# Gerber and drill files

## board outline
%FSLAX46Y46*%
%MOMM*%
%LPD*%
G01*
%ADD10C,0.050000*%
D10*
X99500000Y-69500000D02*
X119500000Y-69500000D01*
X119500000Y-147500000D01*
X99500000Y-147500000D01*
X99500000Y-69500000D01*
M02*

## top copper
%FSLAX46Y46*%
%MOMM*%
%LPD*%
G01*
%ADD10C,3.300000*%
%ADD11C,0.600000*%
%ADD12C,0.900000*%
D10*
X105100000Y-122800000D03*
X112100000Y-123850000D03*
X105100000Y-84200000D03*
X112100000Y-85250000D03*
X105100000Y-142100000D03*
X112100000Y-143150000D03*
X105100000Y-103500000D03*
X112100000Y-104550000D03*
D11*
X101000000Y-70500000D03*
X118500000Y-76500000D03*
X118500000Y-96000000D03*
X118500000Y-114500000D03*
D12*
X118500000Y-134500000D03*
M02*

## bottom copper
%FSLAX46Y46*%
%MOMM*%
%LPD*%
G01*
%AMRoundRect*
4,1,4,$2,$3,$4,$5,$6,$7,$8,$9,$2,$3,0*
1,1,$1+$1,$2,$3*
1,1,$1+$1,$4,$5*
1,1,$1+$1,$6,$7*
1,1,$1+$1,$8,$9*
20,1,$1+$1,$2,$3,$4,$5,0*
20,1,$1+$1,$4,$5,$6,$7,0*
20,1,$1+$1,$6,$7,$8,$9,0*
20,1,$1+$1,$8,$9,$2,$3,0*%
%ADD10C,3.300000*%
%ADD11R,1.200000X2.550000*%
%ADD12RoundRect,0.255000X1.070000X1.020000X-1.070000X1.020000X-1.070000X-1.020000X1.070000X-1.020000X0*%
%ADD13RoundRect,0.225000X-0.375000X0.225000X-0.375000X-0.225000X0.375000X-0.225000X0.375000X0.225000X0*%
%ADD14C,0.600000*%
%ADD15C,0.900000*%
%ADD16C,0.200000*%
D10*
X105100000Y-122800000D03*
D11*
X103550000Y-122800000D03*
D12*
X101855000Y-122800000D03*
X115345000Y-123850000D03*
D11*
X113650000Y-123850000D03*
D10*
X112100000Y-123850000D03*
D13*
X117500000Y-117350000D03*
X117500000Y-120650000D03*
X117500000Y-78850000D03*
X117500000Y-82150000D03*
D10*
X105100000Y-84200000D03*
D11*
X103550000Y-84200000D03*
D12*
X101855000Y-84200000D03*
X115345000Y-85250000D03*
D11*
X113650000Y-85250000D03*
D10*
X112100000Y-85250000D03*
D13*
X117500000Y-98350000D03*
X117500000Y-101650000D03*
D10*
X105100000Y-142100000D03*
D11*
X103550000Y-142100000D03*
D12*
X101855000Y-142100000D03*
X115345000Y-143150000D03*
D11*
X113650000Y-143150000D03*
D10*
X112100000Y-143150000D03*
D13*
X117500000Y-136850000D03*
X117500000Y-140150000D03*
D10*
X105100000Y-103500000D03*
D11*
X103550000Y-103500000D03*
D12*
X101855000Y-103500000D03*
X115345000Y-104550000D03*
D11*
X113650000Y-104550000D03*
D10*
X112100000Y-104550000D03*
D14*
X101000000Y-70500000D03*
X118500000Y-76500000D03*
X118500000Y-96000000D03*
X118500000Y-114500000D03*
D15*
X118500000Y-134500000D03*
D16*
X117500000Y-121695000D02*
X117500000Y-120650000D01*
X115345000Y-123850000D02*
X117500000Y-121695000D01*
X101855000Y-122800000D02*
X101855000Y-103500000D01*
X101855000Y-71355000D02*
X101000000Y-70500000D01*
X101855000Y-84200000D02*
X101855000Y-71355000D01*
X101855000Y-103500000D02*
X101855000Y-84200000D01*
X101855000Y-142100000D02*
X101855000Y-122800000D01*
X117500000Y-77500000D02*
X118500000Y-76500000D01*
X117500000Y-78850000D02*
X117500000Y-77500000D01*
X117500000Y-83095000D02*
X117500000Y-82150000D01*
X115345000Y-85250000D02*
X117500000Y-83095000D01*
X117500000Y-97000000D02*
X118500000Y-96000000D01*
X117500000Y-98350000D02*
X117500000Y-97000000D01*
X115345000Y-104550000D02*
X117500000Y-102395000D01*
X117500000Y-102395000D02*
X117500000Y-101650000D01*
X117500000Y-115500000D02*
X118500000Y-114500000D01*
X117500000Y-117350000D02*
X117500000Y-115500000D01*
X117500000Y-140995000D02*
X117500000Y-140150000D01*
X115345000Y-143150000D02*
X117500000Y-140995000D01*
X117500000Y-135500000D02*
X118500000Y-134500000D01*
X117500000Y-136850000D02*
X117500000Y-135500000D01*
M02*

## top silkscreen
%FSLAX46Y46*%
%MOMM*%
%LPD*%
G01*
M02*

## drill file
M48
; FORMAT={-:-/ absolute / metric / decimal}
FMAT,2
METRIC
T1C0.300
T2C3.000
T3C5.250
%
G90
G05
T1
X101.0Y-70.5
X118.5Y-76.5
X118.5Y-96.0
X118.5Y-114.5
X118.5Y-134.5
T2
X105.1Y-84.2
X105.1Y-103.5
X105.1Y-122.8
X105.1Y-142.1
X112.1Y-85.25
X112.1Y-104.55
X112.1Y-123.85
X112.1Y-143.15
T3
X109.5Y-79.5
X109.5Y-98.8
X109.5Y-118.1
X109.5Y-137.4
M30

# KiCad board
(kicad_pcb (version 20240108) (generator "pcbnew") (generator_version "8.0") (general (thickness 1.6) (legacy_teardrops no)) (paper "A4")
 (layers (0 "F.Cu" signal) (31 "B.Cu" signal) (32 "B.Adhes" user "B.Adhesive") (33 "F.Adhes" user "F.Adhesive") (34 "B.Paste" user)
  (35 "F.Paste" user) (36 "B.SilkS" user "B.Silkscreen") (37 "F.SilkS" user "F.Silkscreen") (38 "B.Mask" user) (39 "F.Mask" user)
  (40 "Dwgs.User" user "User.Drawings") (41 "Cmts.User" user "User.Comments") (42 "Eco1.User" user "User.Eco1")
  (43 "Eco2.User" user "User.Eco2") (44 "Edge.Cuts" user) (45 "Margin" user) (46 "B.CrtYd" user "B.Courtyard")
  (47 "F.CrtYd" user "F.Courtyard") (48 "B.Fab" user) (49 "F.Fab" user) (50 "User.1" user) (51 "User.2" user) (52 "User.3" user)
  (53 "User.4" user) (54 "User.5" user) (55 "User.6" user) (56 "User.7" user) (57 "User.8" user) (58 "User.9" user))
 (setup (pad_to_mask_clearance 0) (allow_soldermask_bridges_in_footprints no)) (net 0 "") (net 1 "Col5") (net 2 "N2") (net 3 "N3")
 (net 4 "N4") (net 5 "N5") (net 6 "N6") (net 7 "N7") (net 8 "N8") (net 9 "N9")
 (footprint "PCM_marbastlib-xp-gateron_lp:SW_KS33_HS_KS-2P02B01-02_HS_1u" (layer "B.Cu") (at 109.5 118.1 180)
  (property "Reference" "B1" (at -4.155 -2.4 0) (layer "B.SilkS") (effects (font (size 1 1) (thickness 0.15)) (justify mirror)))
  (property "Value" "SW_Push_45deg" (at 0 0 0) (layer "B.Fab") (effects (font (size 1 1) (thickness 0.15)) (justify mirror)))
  (pad "" np_thru_hole circle (at 0 0) (size 5.25 5.25) (drill 5.25) (layers "F&B.Cu" "*.Mask"))
  (pad "1" thru_hole circle (at 4.4 -4.7 180) (size 3.3 3.3) (drill 3) (layers "*.Cu" "B.Mask") (remove_unused_layers no) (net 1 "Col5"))
  (pad "1" smd rect (at 5.95 -4.7 180) (size 1.2 2.55) (layers "B.Cu") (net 1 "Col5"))
  (pad "1" smd roundrect (at 7.645 -4.7 180) (size 2.65 2.55) (layers "B.Cu" "B.Paste" "B.Mask") (roundrect_rratio 0.1) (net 1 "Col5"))
  (pad "2" smd roundrect (at -5.845 -5.75 180) (size 2.65 2.55) (layers "B.Cu" "B.Paste" "B.Mask") (roundrect_rratio 0.1) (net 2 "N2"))
  (pad "2" smd rect (at -4.15 -5.75) (size 1.2 2.55) (layers "B.Cu") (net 2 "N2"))
  (pad "2" thru_hole circle (at -2.6 -5.75 180) (size 3.3 3.3) (drill 3) (layers "*.Cu" "B.Mask") (remove_unused_layers no) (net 2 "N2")))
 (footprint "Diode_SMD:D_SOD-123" (layer "B.Cu") (at 117.5 119 -90)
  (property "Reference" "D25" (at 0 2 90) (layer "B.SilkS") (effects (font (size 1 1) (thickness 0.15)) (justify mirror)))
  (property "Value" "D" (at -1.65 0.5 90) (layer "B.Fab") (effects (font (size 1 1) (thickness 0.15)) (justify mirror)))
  (pad "1" smd roundrect (at -1.65 0 270) (size 0.9 1.2) (layers "B.Cu" "B.Paste" "B.Mask") (roundrect_rratio 0.25) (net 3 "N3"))
  (pad "2" smd roundrect (at 1.65 0 270) (size 0.9 1.2) (layers "B.Cu" "B.Paste" "B.Mask") (roundrect_rratio 0.25) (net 2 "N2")))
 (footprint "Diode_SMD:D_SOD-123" (layer "B.Cu") (at 117.5 80.5 -90)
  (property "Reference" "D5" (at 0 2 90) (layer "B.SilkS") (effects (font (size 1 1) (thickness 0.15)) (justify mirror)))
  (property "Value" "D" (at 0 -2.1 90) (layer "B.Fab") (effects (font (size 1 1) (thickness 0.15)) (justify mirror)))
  (pad "1" smd roundrect (at -1.65 0 270) (size 0.9 1.2) (layers "B.Cu" "B.Paste" "B.Mask") (roundrect_rratio 0.25) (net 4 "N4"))
  (pad "2" smd roundrect (at 1.65 0 270) (size 0.9 1.2) (layers "B.Cu" "B.Paste" "B.Mask") (roundrect_rratio 0.25) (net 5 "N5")))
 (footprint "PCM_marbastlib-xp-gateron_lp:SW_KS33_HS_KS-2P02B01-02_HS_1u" (layer "B.Cu") (at 109.5 79.5 180)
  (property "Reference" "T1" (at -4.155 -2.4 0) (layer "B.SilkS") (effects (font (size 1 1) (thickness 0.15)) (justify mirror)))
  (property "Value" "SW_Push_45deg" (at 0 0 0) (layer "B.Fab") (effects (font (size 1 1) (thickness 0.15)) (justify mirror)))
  (pad "" np_thru_hole circle (at 0 0) (size 5.25 5.25) (drill 5.25) (layers "F&B.Cu" "*.Mask"))
  (pad "1" thru_hole circle (at 4.4 -4.7 180) (size 3.3 3.3) (drill 3) (layers "*.Cu" "B.Mask") (remove_unused_layers no) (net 1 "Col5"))
  (pad "1" smd rect (at 5.95 -4.7 180) (size 1.2 2.55) (layers "B.Cu") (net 1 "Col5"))
  (pad "1" smd roundrect (at 7.645 -4.7 180) (size 2.65 2.55) (layers "B.Cu" "B.Paste" "B.Mask") (roundrect_rratio 0.1) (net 1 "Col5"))
  (pad "2" smd roundrect (at -5.845 -5.75 180) (size 2.65 2.55) (layers "B.Cu" "B.Paste" "B.Mask") (roundrect_rratio 0.1) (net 5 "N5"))
  (pad "2" smd rect (at -4.15 -5.75) (size 1.2 2.55) (layers "B.Cu") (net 5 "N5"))
  (pad "2" thru_hole circle (at -2.6 -5.75 180) (size 3.3 3.3) (drill 3) (layers "*.Cu" "B.Mask") (remove_unused_layers no) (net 5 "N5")))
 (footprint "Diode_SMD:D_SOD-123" (layer "B.Cu") (at 117.5 100 -90)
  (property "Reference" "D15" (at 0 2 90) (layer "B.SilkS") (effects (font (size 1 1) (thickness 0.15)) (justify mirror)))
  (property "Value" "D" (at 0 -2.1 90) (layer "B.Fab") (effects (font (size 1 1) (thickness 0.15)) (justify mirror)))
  (pad "1" smd roundrect (at -1.65 0 270) (size 0.9 1.2) (layers "B.Cu" "B.Paste" "B.Mask") (roundrect_rratio 0.25) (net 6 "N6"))
  (pad "2" smd roundrect (at 1.65 0 270) (size 0.9 1.2) (layers "B.Cu" "B.Paste" "B.Mask") (roundrect_rratio 0.25) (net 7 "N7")))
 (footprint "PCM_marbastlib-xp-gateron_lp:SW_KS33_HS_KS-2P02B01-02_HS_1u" (layer "B.Cu") (at 109.5 137.4 180)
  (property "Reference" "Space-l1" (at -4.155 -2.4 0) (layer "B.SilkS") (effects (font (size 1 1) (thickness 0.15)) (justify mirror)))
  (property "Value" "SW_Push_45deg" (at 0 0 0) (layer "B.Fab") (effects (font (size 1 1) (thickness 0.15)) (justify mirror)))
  (pad "" np_thru_hole circle (at 0 0) (size 5.25 5.25) (drill 5.25) (layers "F&B.Cu" "*.Mask"))
  (pad "1" thru_hole circle (at 4.4 -4.7 180) (size 3.3 3.3) (drill 3) (layers "*.Cu" "B.Mask") (remove_unused_layers no) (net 1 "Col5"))
  (pad "1" smd rect (at 5.95 -4.7 180) (size 1.2 2.55) (layers "B.Cu") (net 1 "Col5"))
  (pad "1" smd roundrect (at 7.645 -4.7 180) (size 2.65 2.55) (layers "B.Cu" "B.Paste" "B.Mask") (roundrect_rratio 0.1) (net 1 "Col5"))
  (pad "2" smd roundrect (at -5.845 -5.75 180) (size 2.65 2.55) (layers "B.Cu" "B.Paste" "B.Mask") (roundrect_rratio 0.1) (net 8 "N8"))
  (pad "2" smd rect (at -4.15 -5.75) (size 1.2 2.55) (layers "B.Cu") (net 8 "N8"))
  (pad "2" thru_hole circle (at -2.6 -5.75 180) (size 3.3 3.3) (drill 3) (layers "*.Cu" "B.Mask") (remove_unused_layers no) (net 8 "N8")))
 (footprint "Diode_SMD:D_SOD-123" (layer "B.Cu") (at 117.5 138.5 -90)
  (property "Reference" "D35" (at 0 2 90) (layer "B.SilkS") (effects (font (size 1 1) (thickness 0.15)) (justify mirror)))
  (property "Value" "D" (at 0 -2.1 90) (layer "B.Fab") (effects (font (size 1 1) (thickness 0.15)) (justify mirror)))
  (pad "1" smd roundrect (at -1.65 0 270) (size 0.9 1.2) (layers "B.Cu" "B.Paste" "B.Mask") (roundrect_rratio 0.25) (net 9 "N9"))
  (pad "2" smd roundrect (at 1.65 0 270) (size 0.9 1.2) (layers "B.Cu" "B.Paste" "B.Mask") (roundrect_rratio 0.25) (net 8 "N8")))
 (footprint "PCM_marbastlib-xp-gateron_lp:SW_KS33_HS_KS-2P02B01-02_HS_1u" (layer "B.Cu") (at 109.5 98.8 180)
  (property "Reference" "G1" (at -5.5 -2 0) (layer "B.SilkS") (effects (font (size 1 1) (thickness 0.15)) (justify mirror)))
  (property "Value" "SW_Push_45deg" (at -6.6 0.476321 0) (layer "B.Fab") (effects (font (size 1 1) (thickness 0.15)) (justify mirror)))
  (pad "" np_thru_hole circle (at 0 0) (size 5.25 5.25) (drill 5.25) (layers "F&B.Cu" "*.Mask"))
  (pad "1" thru_hole circle (at 4.4 -4.7 180) (size 3.3 3.3) (drill 3) (layers "*.Cu" "B.Mask") (remove_unused_layers no) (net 1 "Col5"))
  (pad "1" smd rect (at 5.95 -4.7 180) (size 1.2 2.55) (layers "B.Cu") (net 1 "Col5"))
  (pad "1" smd roundrect (at 7.645 -4.7 180) (size 2.65 2.55) (layers "B.Cu" "B.Paste" "B.Mask") (roundrect_rratio 0.1) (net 1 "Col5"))
  (pad "2" smd roundrect (at -5.845 -5.75 180) (size 2.65 2.55) (layers "B.Cu" "B.Paste" "B.Mask") (roundrect_rratio 0.1) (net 7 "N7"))
  (pad "2" smd rect (at -4.15 -5.75) (size 1.2 2.55) (layers "B.Cu") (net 7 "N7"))
  (pad "2" thru_hole circle (at -2.6 -5.75 180) (size 3.3 3.3) (drill 3) (layers "*.Cu" "B.Mask") (remove_unused_layers no) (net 7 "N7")))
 (gr_rect (start 99.5 69.5) (end 119.5 147.5) (stroke (width 0.05) (type default)) (fill none) (layer "Edge.Cuts"))
 (segment (start 117.5 121.695) (end 117.5 120.65) (width 0.2) (layer "B.Cu") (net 2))
 (segment (start 115.345 123.85) (end 117.5 121.695) (width 0.2) (layer "B.Cu") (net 2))
 (via (at 101 70.5) (size 0.6) (drill 0.3) (layers "F.Cu" "B.Cu") (free yes) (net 1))
 (segment (start 101.855 122.8) (end 101.855 103.5) (width 0.2) (layer "B.Cu") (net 1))
 (segment (start 101.855 71.355) (end 101 70.5) (width 0.2) (layer "B.Cu") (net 1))
 (segment (start 101.855 84.2) (end 101.855 71.355) (width 0.2) (layer "B.Cu") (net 1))
 (segment (start 101.855 103.5) (end 101.855 84.2) (width 0.2) (layer "B.Cu") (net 1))
 (segment (start 101.855 142.1) (end 101.855 122.8) (width 0.2) (layer "B.Cu") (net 1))
 (via (at 118.5 76.5) (size 0.6) (drill 0.3) (layers "F.Cu" "B.Cu") (free yes) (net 4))
 (segment (start 117.5 77.5) (end 118.5 76.5) (width 0.2) (layer "B.Cu") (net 4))
 (segment (start 117.5 78.85) (end 117.5 77.5) (width 0.2) (layer "B.Cu") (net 4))
 (segment (start 117.5 83.095) (end 117.5 82.15) (width 0.2) (layer "B.Cu") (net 5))
 (segment (start 115.345 85.25) (end 117.5 83.095) (width 0.2) (layer "B.Cu") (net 5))
 (via (at 118.5 96) (size 0.6) (drill 0.3) (layers "F.Cu" "B.Cu") (free yes) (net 6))
 (segment (start 117.5 97) (end 118.5 96) (width 0.2) (layer "B.Cu") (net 6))
 (segment (start 117.5 98.35) (end 117.5 97) (width 0.2) (layer "B.Cu") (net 6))
 (segment (start 115.345 104.55) (end 117.5 102.395) (width 0.2) (layer "B.Cu") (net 7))
 (segment (start 117.5 102.395) (end 117.5 101.65) (width 0.2) (layer "B.Cu") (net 7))
 (via (at 118.5 114.5) (size 0.6) (drill 0.3) (layers "F.Cu" "B.Cu") (free yes) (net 3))
 (segment (start 117.5 115.5) (end 118.5 114.5) (width 0.2) (layer "B.Cu") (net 3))
 (segment (start 117.5 117.35) (end 117.5 115.5) (width 0.2) (layer "B.Cu") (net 3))
 (segment (start 117.5 140.995) (end 117.5 140.15) (width 0.2) (layer "B.Cu") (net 8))
 (segment (start 115.345 143.15) (end 117.5 140.995) (width 0.2) (layer "B.Cu") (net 8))
 (via (at 118.5 134.5) (size 0.9) (drill 0.3) (layers "F.Cu" "B.Cu") (free yes) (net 9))
 (segment (start 117.5 135.5) (end 118.5 134.5) (width 0.2) (layer "B.Cu") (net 9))
 (segment (start 117.5 136.85) (end 117.5 135.5) (width 0.2) (layer "B.Cu") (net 9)))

